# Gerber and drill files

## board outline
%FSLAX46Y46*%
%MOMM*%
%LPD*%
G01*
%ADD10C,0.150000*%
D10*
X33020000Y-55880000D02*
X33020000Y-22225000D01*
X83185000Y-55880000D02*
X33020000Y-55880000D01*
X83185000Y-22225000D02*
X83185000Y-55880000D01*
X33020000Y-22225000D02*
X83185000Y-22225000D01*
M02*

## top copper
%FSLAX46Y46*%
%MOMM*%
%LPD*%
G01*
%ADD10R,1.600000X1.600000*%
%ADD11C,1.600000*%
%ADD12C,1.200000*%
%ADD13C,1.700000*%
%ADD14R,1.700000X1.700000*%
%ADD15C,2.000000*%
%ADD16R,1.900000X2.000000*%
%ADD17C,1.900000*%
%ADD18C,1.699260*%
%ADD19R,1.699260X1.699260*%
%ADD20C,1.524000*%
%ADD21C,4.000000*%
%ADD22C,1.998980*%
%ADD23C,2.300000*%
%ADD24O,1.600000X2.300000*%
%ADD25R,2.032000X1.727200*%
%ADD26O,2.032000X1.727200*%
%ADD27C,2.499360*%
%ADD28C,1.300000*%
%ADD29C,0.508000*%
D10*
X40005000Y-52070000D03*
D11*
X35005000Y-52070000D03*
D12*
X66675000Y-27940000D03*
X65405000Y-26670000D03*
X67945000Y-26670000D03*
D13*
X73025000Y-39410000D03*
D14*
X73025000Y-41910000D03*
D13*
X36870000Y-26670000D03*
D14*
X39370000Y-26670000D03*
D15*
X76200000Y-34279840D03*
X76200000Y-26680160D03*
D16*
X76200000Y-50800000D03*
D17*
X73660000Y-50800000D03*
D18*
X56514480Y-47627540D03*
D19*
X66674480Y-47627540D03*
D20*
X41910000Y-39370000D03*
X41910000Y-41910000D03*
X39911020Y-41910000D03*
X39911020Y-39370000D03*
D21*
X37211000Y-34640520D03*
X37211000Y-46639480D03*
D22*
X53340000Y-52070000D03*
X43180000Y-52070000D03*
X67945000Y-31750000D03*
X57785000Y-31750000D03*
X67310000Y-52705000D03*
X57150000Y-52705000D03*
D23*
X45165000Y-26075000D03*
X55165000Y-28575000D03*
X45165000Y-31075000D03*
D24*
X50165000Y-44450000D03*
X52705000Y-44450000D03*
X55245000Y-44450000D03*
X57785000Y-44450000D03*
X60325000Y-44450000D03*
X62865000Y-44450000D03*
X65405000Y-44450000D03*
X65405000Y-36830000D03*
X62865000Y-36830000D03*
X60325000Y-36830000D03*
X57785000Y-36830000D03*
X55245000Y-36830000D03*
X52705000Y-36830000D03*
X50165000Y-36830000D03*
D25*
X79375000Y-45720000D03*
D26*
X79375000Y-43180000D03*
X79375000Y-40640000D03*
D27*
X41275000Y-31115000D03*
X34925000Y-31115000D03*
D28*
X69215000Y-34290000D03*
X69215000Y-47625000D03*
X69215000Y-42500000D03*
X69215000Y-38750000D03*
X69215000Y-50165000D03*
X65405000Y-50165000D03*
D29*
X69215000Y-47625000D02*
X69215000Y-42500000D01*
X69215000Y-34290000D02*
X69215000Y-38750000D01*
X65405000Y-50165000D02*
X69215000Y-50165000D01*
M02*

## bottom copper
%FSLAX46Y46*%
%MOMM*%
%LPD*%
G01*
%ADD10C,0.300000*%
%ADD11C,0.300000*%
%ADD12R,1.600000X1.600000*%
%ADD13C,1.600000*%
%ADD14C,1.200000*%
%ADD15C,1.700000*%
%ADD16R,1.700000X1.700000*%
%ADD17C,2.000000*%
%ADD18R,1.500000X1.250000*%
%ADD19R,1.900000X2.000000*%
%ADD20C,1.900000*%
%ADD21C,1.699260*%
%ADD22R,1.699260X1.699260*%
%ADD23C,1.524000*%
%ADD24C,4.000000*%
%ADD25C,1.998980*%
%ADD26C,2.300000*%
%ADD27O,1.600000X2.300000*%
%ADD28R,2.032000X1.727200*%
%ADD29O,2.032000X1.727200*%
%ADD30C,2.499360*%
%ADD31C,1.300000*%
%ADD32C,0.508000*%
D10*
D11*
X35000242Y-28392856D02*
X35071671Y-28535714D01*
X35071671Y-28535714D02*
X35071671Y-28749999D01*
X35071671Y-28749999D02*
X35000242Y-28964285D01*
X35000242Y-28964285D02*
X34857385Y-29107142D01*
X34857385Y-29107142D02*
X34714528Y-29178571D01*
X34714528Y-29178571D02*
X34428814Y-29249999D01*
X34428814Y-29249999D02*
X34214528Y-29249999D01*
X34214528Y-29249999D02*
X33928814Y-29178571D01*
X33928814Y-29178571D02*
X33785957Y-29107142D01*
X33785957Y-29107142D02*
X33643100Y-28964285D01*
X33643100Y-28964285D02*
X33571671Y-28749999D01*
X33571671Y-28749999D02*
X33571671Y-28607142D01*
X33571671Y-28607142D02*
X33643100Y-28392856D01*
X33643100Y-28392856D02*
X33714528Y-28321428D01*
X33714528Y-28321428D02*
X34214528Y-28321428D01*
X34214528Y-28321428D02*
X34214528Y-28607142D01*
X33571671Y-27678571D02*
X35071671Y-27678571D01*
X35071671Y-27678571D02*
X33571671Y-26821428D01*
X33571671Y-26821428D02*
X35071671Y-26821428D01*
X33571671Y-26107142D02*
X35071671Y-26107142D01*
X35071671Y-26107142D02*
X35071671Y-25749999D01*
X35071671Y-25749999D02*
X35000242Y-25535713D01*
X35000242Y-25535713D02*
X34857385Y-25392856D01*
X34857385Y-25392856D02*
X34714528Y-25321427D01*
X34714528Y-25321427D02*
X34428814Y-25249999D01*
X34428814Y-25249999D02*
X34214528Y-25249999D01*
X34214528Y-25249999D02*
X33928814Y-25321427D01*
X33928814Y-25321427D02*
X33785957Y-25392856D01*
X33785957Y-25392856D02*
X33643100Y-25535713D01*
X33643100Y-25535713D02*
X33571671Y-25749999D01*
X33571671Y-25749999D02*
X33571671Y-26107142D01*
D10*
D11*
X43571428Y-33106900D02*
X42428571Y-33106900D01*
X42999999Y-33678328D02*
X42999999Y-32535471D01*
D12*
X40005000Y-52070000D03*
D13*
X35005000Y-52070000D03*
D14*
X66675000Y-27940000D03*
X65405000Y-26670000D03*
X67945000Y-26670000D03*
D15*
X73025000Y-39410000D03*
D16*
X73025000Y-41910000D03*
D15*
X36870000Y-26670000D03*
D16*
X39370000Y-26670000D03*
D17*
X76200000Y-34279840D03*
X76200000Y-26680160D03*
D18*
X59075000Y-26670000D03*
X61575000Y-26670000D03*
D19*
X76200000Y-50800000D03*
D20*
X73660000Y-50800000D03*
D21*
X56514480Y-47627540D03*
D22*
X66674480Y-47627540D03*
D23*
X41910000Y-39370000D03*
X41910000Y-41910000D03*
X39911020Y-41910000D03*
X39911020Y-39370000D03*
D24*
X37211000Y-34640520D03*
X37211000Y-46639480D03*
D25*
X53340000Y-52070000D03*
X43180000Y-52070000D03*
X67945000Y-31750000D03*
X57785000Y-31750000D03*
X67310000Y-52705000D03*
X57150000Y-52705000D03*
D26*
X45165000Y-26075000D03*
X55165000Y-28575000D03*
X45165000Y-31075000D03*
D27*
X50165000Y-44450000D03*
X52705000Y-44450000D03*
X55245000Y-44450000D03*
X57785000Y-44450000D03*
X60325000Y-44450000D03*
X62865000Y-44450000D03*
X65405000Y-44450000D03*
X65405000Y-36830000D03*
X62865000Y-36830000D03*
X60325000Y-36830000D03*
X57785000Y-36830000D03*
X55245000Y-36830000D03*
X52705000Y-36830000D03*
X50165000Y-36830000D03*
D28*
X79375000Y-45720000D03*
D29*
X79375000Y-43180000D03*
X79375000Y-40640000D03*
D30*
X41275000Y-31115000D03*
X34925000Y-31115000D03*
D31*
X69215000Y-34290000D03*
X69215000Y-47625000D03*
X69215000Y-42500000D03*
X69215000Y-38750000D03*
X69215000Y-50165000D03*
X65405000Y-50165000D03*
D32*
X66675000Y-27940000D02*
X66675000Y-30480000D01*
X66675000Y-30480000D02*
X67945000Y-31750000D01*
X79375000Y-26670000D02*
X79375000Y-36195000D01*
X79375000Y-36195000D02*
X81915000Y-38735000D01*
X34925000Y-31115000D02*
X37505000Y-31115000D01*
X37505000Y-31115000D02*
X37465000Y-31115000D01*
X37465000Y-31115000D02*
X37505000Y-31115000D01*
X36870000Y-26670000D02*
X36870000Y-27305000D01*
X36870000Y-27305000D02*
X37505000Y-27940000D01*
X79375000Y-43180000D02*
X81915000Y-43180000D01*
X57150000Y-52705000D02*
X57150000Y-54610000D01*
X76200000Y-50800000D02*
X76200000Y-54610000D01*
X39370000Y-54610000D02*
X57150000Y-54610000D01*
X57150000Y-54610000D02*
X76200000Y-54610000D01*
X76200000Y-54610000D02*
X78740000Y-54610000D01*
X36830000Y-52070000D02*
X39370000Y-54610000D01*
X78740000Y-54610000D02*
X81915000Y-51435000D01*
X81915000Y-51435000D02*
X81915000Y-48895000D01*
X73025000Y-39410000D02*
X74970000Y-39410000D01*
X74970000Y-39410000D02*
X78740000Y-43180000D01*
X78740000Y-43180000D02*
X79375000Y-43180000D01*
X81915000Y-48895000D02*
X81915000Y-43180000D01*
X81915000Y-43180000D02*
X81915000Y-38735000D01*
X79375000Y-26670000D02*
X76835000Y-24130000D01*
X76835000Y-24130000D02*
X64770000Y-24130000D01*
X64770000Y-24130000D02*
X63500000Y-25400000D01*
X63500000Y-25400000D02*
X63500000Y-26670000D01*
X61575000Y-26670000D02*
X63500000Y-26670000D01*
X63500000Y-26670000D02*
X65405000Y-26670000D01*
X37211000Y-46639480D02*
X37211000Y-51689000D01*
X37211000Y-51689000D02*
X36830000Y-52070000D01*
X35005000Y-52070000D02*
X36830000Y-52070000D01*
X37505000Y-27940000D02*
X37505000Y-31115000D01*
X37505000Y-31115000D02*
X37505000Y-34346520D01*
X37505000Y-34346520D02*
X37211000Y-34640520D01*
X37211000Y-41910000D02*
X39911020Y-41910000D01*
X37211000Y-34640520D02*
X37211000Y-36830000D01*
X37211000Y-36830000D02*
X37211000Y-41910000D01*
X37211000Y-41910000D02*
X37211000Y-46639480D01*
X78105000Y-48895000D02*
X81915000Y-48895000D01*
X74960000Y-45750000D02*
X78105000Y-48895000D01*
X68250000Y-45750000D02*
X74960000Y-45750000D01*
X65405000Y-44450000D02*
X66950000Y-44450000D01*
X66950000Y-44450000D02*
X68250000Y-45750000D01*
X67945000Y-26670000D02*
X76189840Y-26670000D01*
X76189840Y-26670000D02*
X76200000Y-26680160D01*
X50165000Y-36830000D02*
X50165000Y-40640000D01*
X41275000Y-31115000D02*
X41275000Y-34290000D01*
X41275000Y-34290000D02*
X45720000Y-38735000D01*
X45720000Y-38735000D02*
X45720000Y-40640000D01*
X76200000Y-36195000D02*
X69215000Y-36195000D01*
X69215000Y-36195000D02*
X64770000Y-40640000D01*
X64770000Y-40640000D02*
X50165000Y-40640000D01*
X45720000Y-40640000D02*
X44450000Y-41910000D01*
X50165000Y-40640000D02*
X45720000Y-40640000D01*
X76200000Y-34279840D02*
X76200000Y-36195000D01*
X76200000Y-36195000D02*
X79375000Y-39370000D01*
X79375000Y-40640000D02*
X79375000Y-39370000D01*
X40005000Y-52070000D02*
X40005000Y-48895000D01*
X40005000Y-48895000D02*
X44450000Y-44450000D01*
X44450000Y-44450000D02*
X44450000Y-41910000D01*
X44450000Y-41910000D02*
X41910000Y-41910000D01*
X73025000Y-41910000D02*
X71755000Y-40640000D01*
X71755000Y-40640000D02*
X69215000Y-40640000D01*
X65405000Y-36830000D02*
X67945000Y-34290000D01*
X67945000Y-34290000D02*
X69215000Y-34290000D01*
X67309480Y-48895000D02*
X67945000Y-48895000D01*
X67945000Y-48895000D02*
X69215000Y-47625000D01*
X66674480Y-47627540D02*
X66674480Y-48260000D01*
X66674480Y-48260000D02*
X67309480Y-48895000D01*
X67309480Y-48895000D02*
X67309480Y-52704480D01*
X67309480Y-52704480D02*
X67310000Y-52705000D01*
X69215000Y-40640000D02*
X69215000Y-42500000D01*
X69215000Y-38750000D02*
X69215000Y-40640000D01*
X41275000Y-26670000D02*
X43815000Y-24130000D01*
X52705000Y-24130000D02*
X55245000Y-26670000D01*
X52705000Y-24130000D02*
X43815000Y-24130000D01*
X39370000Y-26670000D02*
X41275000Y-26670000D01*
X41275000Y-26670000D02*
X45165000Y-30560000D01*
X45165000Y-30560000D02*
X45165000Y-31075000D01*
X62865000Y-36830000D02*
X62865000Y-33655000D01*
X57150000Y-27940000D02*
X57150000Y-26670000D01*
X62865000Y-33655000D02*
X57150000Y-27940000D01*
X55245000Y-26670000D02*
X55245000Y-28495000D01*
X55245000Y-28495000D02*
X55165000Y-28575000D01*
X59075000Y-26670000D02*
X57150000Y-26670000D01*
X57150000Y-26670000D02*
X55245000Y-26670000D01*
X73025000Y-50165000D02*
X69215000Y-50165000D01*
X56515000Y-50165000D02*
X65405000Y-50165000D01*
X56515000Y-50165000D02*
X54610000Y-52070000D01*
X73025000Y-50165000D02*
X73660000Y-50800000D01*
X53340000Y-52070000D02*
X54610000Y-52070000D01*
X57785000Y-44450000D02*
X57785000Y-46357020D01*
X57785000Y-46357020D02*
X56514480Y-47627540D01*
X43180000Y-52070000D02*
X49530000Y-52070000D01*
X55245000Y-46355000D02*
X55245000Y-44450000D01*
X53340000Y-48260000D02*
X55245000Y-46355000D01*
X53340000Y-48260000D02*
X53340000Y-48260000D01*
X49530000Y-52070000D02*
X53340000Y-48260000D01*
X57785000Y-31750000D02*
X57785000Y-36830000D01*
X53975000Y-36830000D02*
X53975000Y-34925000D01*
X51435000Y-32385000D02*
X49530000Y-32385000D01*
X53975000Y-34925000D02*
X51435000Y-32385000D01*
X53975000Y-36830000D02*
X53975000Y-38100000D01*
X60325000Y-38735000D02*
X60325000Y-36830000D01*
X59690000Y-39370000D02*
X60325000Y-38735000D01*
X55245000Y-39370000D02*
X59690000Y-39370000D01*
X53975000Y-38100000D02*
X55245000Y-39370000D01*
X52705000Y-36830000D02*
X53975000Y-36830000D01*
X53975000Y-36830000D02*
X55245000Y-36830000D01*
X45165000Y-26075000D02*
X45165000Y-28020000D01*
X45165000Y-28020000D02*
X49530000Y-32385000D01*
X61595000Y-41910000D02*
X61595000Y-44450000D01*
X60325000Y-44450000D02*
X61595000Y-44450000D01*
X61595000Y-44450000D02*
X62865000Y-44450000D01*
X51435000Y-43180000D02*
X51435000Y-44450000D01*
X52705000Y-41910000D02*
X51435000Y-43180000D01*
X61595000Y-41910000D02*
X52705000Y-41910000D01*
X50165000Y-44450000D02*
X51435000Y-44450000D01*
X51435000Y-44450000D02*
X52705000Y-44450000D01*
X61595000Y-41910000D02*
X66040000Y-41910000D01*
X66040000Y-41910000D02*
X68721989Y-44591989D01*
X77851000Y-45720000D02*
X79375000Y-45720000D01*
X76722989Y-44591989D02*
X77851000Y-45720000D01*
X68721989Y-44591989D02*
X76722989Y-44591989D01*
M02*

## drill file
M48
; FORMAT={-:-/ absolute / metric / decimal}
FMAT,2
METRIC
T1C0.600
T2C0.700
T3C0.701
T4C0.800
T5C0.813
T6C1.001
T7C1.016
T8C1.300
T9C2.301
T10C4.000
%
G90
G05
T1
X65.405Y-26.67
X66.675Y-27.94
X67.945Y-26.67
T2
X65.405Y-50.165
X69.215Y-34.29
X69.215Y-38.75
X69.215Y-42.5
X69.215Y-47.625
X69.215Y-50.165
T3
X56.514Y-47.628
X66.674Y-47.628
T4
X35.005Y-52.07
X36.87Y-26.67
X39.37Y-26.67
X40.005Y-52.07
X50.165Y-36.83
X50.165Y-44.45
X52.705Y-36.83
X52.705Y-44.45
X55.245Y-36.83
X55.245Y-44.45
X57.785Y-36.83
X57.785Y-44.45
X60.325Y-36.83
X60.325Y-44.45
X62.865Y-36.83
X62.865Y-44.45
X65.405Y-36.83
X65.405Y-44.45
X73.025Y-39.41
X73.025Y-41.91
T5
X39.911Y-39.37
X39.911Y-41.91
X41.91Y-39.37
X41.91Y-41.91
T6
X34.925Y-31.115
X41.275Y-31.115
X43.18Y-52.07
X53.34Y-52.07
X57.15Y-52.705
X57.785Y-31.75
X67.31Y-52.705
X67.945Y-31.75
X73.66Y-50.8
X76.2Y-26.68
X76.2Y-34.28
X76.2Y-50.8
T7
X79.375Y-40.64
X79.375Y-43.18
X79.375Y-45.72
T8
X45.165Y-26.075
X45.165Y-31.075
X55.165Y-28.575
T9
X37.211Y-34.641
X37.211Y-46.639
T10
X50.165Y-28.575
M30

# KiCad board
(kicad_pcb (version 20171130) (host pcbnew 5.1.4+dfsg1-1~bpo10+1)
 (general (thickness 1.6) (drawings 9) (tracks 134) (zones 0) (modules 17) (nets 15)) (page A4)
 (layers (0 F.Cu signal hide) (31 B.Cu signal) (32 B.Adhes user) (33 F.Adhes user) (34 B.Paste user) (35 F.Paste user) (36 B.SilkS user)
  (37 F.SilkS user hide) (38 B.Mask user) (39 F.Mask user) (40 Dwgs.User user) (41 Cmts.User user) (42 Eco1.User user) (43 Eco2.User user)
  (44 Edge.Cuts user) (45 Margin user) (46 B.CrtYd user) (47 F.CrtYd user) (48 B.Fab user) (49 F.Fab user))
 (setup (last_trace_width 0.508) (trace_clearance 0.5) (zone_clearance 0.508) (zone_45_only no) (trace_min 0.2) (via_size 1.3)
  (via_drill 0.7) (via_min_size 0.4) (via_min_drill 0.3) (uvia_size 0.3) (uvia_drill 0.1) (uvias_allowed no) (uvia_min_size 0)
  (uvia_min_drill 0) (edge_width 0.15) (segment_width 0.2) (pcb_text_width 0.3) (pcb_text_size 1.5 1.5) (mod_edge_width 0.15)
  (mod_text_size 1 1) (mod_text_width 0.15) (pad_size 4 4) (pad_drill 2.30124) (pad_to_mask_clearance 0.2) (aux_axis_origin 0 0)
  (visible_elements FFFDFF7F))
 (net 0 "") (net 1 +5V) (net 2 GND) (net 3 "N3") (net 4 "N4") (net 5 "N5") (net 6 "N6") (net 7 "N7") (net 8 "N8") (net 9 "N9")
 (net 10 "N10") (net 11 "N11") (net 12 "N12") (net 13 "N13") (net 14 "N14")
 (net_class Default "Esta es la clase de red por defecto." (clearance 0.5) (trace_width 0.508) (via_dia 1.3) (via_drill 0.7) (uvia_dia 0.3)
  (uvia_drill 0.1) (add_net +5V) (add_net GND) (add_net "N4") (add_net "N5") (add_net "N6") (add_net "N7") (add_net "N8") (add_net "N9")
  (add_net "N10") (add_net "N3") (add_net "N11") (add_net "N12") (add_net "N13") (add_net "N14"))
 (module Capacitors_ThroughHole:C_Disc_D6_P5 (layer F.Cu) (at 40.005 52.07 180)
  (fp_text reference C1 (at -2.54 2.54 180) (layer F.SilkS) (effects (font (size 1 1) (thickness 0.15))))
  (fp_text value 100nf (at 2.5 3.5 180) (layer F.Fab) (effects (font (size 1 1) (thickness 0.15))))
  (pad 1 thru_hole rect (at 0 0 180) (size 1.6 1.6) (drill 0.8) (layers *.Cu *.Mask F.SilkS) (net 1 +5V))
  (pad 2 thru_hole circle (at 5 0 180) (size 1.6 1.6) (drill 0.8) (layers *.Cu *.Mask F.SilkS) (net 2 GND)))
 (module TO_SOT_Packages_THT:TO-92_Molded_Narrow (layer F.Cu) (at 67.945 26.67 180)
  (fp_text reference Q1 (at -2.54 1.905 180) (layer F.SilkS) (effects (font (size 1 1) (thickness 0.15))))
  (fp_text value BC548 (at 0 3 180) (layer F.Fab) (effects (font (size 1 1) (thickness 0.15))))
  (pad 2 thru_hole circle (at 1.27 -1.27 270) (size 1.2 1.2) (drill 0.6) (layers *.Cu *.Mask F.SilkS) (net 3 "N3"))
  (pad 3 thru_hole circle (at 2.54 0 270) (size 1.2 1.2) (drill 0.6) (layers *.Cu *.Mask F.SilkS) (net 2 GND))
  (pad 1 thru_hole circle (at 0 0 270) (size 1.2 1.2) (drill 0.6) (layers *.Cu *.Mask F.SilkS) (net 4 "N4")))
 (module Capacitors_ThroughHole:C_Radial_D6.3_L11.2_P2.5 (layer F.Cu) (at 73.025 41.91 90)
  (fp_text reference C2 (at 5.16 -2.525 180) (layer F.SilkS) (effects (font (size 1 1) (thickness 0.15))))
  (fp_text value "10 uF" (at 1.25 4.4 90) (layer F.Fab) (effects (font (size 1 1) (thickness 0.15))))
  (pad 2 thru_hole circle (at 2.5 0 90) (size 1.7 1.7) (drill 0.8) (layers *.Cu *.Mask F.SilkS) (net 2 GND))
  (pad 1 thru_hole rect (at 0 0 90) (size 1.7 1.7) (drill 0.8) (layers *.Cu *.Mask F.SilkS) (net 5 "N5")))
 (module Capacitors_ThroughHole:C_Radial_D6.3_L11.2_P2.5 (layer F.Cu) (at 39.37 26.67 180)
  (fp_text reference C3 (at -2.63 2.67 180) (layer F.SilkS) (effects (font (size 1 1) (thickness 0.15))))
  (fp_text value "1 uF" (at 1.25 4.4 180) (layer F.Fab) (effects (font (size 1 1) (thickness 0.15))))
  (pad 2 thru_hole circle (at 2.5 0 180) (size 1.7 1.7) (drill 0.8) (layers *.Cu *.Mask F.SilkS) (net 2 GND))
  (pad 1 thru_hole rect (at 0 0 180) (size 1.7 1.7) (drill 0.8) (layers *.Cu *.Mask F.SilkS) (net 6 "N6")))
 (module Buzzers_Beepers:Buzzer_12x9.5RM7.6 (layer F.Cu) (at 76.2 30.48 90)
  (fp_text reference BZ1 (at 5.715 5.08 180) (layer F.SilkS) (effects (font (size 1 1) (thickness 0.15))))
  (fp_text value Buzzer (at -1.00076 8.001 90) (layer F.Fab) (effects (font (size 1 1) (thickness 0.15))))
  (pad 1 thru_hole circle (at -3.79984 0 90) (size 2 2) (drill 1.00076) (layers *.Cu *.Mask F.SilkS) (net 1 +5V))
  (pad 2 thru_hole circle (at 3.79984 0 90) (size 2 2) (drill 1.00076) (layers *.Cu *.Mask F.SilkS) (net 4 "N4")))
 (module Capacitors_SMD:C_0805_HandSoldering (layer B.Cu) (at 60.325 26.67)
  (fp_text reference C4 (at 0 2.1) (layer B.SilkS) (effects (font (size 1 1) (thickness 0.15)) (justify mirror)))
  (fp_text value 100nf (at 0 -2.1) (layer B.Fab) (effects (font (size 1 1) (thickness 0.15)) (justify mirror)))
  (pad 1 smd rect (at -1.25 0) (size 1.5 1.25) (layers B.Cu B.Paste B.Mask) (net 6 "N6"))
  (pad 2 smd rect (at 1.25 0) (size 1.5 1.25) (layers B.Cu B.Paste B.Mask) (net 2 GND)))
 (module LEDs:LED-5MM (layer F.Cu) (at 76.2 50.8 180)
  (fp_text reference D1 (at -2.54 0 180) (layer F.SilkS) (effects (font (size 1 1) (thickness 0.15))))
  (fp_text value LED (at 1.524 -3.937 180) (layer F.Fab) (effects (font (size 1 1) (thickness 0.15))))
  (pad 1 thru_hole rect (at 0 0 270) (size 2 1.9) (drill 1.00076) (layers *.Cu *.Mask F.SilkS) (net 2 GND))
  (pad 2 thru_hole circle (at 2.54 0 180) (size 1.9 1.9) (drill 1.00076) (layers *.Cu *.Mask F.SilkS) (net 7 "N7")))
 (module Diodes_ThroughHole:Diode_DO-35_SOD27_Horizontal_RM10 (layer F.Cu) (at 66.675 47.625 180)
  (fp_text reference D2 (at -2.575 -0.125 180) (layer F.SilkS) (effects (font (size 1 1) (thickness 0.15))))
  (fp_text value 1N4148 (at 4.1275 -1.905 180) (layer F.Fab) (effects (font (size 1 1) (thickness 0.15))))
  (pad 2 thru_hole circle (at 10.16052 -0.00254) (size 1.69926 1.69926) (drill 0.70104) (layers *.Cu *.Mask F.SilkS) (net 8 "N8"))
  (pad 1 thru_hole rect (at 0.00052 -0.00254) (size 1.69926 1.69926) (drill 0.70104) (layers *.Cu *.Mask F.SilkS) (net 5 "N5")))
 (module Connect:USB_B (layer F.Cu) (at 41.91 41.91 180) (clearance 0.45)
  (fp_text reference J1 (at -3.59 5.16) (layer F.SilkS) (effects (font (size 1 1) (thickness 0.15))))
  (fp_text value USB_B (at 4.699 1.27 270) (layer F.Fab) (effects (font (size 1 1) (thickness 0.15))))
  (pad 2 thru_hole circle (at 0 2.54 90) (size 1.524 1.524) (drill 0.8128) (layers *.Cu *.Mask F.SilkS) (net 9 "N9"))
  (pad 1 thru_hole circle (at 0 0 90) (size 1.524 1.524) (drill 0.8128) (layers *.Cu *.Mask F.SilkS) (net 1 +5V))
  (pad 4 thru_hole circle (at 1.99898 0 90) (size 1.524 1.524) (drill 0.8128) (layers *.Cu *.Mask F.SilkS) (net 2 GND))
  (pad 3 thru_hole circle (at 1.99898 2.54 90) (size 1.524 1.524) (drill 0.8128) (layers *.Cu *.Mask F.SilkS) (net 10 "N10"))
  (pad 5 thru_hole circle (at 4.699 7.26948 90) (size 4 4) (drill 2.30124) (layers *.Cu *.Mask F.SilkS) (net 2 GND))
  (pad 5 thru_hole circle (at 4.699 -4.72948 90) (size 4 4) (drill 2.30124) (layers *.Cu *.Mask F.SilkS) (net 2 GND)))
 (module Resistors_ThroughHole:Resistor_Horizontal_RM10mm (layer F.Cu) (at 53.34 52.07 180)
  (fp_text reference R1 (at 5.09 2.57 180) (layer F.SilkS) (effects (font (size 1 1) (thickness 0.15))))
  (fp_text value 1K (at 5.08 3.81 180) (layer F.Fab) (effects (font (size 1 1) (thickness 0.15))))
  (pad 1 thru_hole circle (at 0 0 180) (size 1.99898 1.99898) (drill 1.00076) (layers *.Cu *.SilkS *.Mask) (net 7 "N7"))
  (pad 2 thru_hole circle (at 10.16 0 180) (size 1.99898 1.99898) (drill 1.00076) (layers *.Cu *.SilkS *.Mask) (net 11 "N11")))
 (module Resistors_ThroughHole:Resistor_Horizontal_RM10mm (layer F.Cu) (at 67.945 31.75 180)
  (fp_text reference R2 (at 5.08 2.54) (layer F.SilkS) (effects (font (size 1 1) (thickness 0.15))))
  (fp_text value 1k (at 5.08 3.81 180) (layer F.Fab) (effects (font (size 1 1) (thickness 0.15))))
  (pad 1 thru_hole circle (at 0 0 180) (size 1.99898 1.99898) (drill 1.00076) (layers *.Cu *.SilkS *.Mask) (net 3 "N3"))
  (pad 2 thru_hole circle (at 10.16 0 180) (size 1.99898 1.99898) (drill 1.00076) (layers *.Cu *.SilkS *.Mask) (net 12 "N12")))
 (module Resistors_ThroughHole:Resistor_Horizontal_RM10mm (layer F.Cu) (at 67.31 52.705 180)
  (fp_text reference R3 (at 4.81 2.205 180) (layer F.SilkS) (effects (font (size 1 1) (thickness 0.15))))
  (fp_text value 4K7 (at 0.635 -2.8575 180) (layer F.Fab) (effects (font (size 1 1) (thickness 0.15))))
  (pad 1 thru_hole circle (at 0 0 180) (size 1.99898 1.99898) (drill 1.00076) (layers *.Cu *.SilkS *.Mask) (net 5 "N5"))
  (pad 2 thru_hole circle (at 10.16 0 180) (size 1.99898 1.99898) (drill 1.00076) (layers *.Cu *.SilkS *.Mask) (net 2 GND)))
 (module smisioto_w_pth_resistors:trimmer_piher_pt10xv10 (layer F.Cu) (at 50.165 28.575 90)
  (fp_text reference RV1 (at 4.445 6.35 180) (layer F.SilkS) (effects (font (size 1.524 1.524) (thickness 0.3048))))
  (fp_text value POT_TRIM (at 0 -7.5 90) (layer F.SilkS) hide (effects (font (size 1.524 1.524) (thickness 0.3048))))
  (pad 1 thru_hole circle (at 2.5 -5 90) (size 2.3 2.3) (drill 1.3) (layers *.Cu *.Mask F.SilkS) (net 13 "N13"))
  (pad 2 thru_hole circle (at 0 5 90) (size 2.3 2.3) (drill 1.3) (layers *.Cu *.Mask F.SilkS) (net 6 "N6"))
  (pad 3 thru_hole circle (at -2.5 -5 90) (size 2.3 2.3) (drill 1.3) (layers *.Cu *.Mask F.SilkS) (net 6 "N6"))
  (pad "" np_thru_hole circle (at 0 0 90) (size 4 4) (drill 4) (layers *.Cu *.Mask F.SilkS)))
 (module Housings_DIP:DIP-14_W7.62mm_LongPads (layer F.Cu) (at 50.165 44.45 90)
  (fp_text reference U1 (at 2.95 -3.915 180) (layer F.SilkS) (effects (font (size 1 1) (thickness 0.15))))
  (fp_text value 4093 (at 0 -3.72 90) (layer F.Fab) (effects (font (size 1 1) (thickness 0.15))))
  (pad 1 thru_hole oval (at 0 0 90) (size 2.3 1.6) (drill 0.8) (layers *.Cu *.Mask F.SilkS) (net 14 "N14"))
  (pad 2 thru_hole oval (at 0 2.54 90) (size 2.3 1.6) (drill 0.8) (layers *.Cu *.Mask F.SilkS) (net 14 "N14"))
  (pad 3 thru_hole oval (at 0 5.08 90) (size 2.3 1.6) (drill 0.8) (layers *.Cu *.Mask F.SilkS) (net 11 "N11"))
  (pad 4 thru_hole oval (at 0 7.62 90) (size 2.3 1.6) (drill 0.8) (layers *.Cu *.Mask F.SilkS) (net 8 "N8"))
  (pad 5 thru_hole oval (at 0 10.16 90) (size 2.3 1.6) (drill 0.8) (layers *.Cu *.Mask F.SilkS) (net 14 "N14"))
  (pad 6 thru_hole oval (at 0 12.7 90) (size 2.3 1.6) (drill 0.8) (layers *.Cu *.Mask F.SilkS) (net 14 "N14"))
  (pad 7 thru_hole oval (at 0 15.24 90) (size 2.3 1.6) (drill 0.8) (layers *.Cu *.Mask F.SilkS) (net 2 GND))
  (pad 8 thru_hole oval (at 7.62 15.24 90) (size 2.3 1.6) (drill 0.8) (layers *.Cu *.Mask F.SilkS) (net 5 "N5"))
  (pad 9 thru_hole oval (at 7.62 12.7 90) (size 2.3 1.6) (drill 0.8) (layers *.Cu *.Mask F.SilkS) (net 6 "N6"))
  (pad 10 thru_hole oval (at 7.62 10.16 90) (size 2.3 1.6) (drill 0.8) (layers *.Cu *.Mask F.SilkS) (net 13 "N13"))
  (pad 11 thru_hole oval (at 7.62 7.62 90) (size 2.3 1.6) (drill 0.8) (layers *.Cu *.Mask F.SilkS) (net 12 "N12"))
  (pad 12 thru_hole oval (at 7.62 5.08 90) (size 2.3 1.6) (drill 0.8) (layers *.Cu *.Mask F.SilkS) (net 13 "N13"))
  (pad 13 thru_hole oval (at 7.62 2.54 90) (size 2.3 1.6) (drill 0.8) (layers *.Cu *.Mask F.SilkS) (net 13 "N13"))
  (pad 14 thru_hole oval (at 7.62 0 90) (size 2.3 1.6) (drill 0.8) (layers *.Cu *.Mask F.SilkS) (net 1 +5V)))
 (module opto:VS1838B (layer F.Cu) (at 79.375 45.72 180)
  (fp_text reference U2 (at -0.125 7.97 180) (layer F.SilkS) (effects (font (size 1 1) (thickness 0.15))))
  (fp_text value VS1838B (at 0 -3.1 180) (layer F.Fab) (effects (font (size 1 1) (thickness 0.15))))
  (pad 1 thru_hole rect (at 0 0 180) (size 2.032 1.7272) (drill 1.016) (layers *.Cu *.Mask F.SilkS) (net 14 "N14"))
  (pad 2 thru_hole oval (at 0 2.54 180) (size 2.032 1.7272) (drill 1.016) (layers *.Cu *.Mask F.SilkS) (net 2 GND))
  (pad 3 thru_hole oval (at 0 5.08 180) (size 2.032 1.7272) (drill 1.016) (layers *.Cu *.Mask F.SilkS) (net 1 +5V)))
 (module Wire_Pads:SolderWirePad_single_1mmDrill (layer F.Cu) (at 41.275 31.115)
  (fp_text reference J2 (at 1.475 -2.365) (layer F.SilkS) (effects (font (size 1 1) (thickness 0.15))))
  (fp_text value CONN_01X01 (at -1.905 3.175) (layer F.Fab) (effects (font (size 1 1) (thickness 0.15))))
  (pad 1 thru_hole circle (at 0 0) (size 2.49936 2.49936) (drill 1.00076) (layers *.Cu *.Mask F.SilkS) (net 1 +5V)))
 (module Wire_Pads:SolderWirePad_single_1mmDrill (layer F.Cu) (at 34.925 31.115)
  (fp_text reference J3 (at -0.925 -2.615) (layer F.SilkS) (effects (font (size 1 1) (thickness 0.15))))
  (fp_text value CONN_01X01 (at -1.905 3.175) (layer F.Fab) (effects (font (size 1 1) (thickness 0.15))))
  (pad 1 thru_hole circle (at 0 0) (size 2.49936 2.49936) (drill 1.00076) (layers *.Cu *.Mask F.SilkS) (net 2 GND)))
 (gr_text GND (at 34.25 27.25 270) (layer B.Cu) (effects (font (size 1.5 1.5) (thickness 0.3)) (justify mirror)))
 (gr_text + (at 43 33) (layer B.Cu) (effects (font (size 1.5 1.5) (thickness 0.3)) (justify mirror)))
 (gr_line (start 33.02 55.88) (end 33.02 22.225) (angle 90) (layer Edge.Cuts) (width 0.15))
 (gr_line (start 83.185 55.88) (end 33.02 55.88) (angle 90) (layer Edge.Cuts) (width 0.15))
 (gr_line (start 83.185 22.225) (end 83.185 55.88) (angle 90) (layer Edge.Cuts) (width 0.15))
 (gr_line (start 33.02 22.225) (end 83.185 22.225) (angle 90) (layer Edge.Cuts) (width 0.15))
 (segment (start 66.675 27.94) (end 66.675 30.48) (width 0.508) (layer B.Cu) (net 3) (status 10))
 (segment (start 66.675 30.48) (end 67.945 31.75) (width 0.508) (layer B.Cu) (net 3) (status 20))
 (segment (start 79.375 26.67) (end 79.375 36.195) (width 0.508) (layer B.Cu) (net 2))
 (segment (start 79.375 36.195) (end 81.915 38.735) (width 0.508) (layer B.Cu) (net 2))
 (segment (start 34.925 31.115) (end 37.505 31.115) (width 0.508) (layer B.Cu) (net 2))
 (segment (start 37.505 31.115) (end 37.465 31.115) (width 0.508) (layer B.Cu) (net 2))
 (segment (start 37.465 31.115) (end 37.505 31.115) (width 0.508) (layer B.Cu) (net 2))
 (segment (start 36.87 26.67) (end 36.87 27.305) (width 0.508) (layer B.Cu) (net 2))
 (segment (start 36.87 27.305) (end 37.505 27.94) (width 0.508) (layer B.Cu) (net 2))
 (segment (start 79.375 43.18) (end 81.915 43.18) (width 0.508) (layer B.Cu) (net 2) (status 10))
 (segment (start 57.15 52.705) (end 57.15 54.61) (width 0.508) (layer B.Cu) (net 2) (status 10))
 (segment (start 76.2 50.8) (end 76.2 54.61) (width 0.508) (layer B.Cu) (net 2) (status 10))
 (segment (start 39.37 54.61) (end 57.15 54.61) (width 0.508) (layer B.Cu) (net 2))
 (segment (start 57.15 54.61) (end 76.2 54.61) (width 0.508) (layer B.Cu) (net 2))
 (segment (start 76.2 54.61) (end 78.74 54.61) (width 0.508) (layer B.Cu) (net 2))
 (segment (start 36.83 52.07) (end 39.37 54.61) (width 0.508) (layer B.Cu) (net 2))
 (segment (start 78.74 54.61) (end 81.915 51.435) (width 0.508) (layer B.Cu) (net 2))
 (segment (start 81.915 51.435) (end 81.915 48.895) (width 0.508) (layer B.Cu) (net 2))
 (segment (start 73.025 39.41) (end 74.97 39.41) (width 0.508) (layer B.Cu) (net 2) (status 10))
 (segment (start 74.97 39.41) (end 78.74 43.18) (width 0.508) (layer B.Cu) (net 2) (status 20))
 (segment (start 78.74 43.18) (end 79.375 43.18) (width 0.508) (layer B.Cu) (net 2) (status 30))
 (segment (start 81.915 48.895) (end 81.915 43.18) (width 0.508) (layer B.Cu) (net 2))
 (segment (start 81.915 43.18) (end 81.915 38.735) (width 0.508) (layer B.Cu) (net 2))
 (segment (start 79.375 26.67) (end 76.835 24.13) (width 0.508) (layer B.Cu) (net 2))
 (segment (start 76.835 24.13) (end 64.77 24.13) (width 0.508) (layer B.Cu) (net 2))
 (segment (start 64.77 24.13) (end 63.5 25.4) (width 0.508) (layer B.Cu) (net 2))
 (segment (start 63.5 25.4) (end 63.5 26.67) (width 0.508) (layer B.Cu) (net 2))
 (segment (start 61.575 26.67) (end 63.5 26.67) (width 0.508) (layer B.Cu) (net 2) (status 10))
 (segment (start 63.5 26.67) (end 65.405 26.67) (width 0.508) (layer B.Cu) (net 2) (status 20))
 (segment (start 37.211 46.63948) (end 37.211 51.689) (width 0.508) (layer B.Cu) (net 2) (status 10))
 (segment (start 37.211 51.689) (end 36.83 52.07) (width 0.508) (layer B.Cu) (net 2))
 (segment (start 35.005 52.07) (end 36.83 52.07) (width 0.508) (layer B.Cu) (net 2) (status 10))
 (segment (start 37.505 27.94) (end 37.505 31.115) (width 0.508) (layer B.Cu) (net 2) (status 30))
 (segment (start 37.505 31.115) (end 37.505 34.34652) (width 0.508) (layer B.Cu) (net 2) (status 30))
 (segment (start 37.505 34.34652) (end 37.211 34.64052) (width 0.508) (layer B.Cu) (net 2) (status 30))
 (segment (start 37.211 41.91) (end 39.91102 41.91) (width 0.508) (layer B.Cu) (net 2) (status 20))
 (segment (start 37.211 34.64052) (end 37.211 36.83) (width 0.508) (layer B.Cu) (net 2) (status 10))
 (segment (start 37.211 36.83) (end 37.211 41.91) (width 0.508) (layer B.Cu) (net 2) (status 10))
 (segment (start 37.211 41.91) (end 37.211 46.63948) (width 0.508) (layer B.Cu) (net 2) (status 20))
 (segment (start 78.105 48.895) (end 81.915 48.895) (width 0.508) (layer B.Cu) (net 2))
 (segment (start 74.96 45.75) (end 78.105 48.895) (width 0.508) (layer B.Cu) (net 2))
 (segment (start 68.25 45.75) (end 74.96 45.75) (width 0.508) (layer B.Cu) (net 2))
 (segment (start 65.405 44.45) (end 66.95 44.45) (width 0.508) (layer B.Cu) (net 2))
 (segment (start 66.95 44.45) (end 68.25 45.75) (width 0.508) (layer B.Cu) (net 2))
 (segment (start 67.945 26.67) (end 76.18984 26.67) (width 0.508) (layer B.Cu) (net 4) (status 30))
 (segment (start 76.18984 26.67) (end 76.2 26.68016) (width 0.508) (layer B.Cu) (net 4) (status 30))
 (segment (start 50.165 36.83) (end 50.165 40.64) (width 0.508) (layer B.Cu) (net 1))
 (segment (start 41.275 31.115) (end 41.275 34.29) (width 0.508) (layer B.Cu) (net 1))
 (segment (start 41.275 34.29) (end 45.72 38.735) (width 0.508) (layer B.Cu) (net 1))
 (segment (start 45.72 38.735) (end 45.72 40.64) (width 0.508) (layer B.Cu) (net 1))
 (segment (start 76.2 36.195) (end 69.215 36.195) (width 0.508) (layer B.Cu) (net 1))
 (segment (start 69.215 36.195) (end 64.77 40.64) (width 0.508) (layer B.Cu) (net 1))
 (segment (start 64.77 40.64) (end 50.165 40.64) (width 0.508) (layer B.Cu) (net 1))
 (segment (start 45.72 40.64) (end 44.45 41.91) (width 0.508) (layer B.Cu) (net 1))
 (segment (start 50.165 40.64) (end 45.72 40.64) (width 0.508) (layer B.Cu) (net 1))
 (segment (start 76.2 34.27984) (end 76.2 36.195) (width 0.508) (layer B.Cu) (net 1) (status 10))
 (segment (start 76.2 36.195) (end 79.375 39.37) (width 0.508) (layer B.Cu) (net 1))
 (segment (start 79.375 40.64) (end 79.375 39.37) (width 0.508) (layer B.Cu) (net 1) (status 10))
 (segment (start 40.005 52.07) (end 40.005 48.895) (width 0.508) (layer B.Cu) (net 1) (status 10))
 (segment (start 40.005 48.895) (end 44.45 44.45) (width 0.508) (layer B.Cu) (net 1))
 (segment (start 44.45 44.45) (end 44.45 41.91) (width 0.508) (layer B.Cu) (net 1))
 (segment (start 44.45 41.91) (end 41.91 41.91) (width 0.508) (layer B.Cu) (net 1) (status 20))
 (segment (start 73.025 41.91) (end 71.755 40.64) (width 0.508) (layer B.Cu) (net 5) (status 10))
 (segment (start 71.755 40.64) (end 69.215 40.64) (width 0.508) (layer B.Cu) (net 5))
 (segment (start 65.405 36.83) (end 67.945 34.29) (width 0.508) (layer B.Cu) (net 5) (status 10))
 (via (at 69.215 34.29) (size 1.3) (drill 0.7) (layers F.Cu B.Cu) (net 5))
 (segment (start 67.945 34.29) (end 69.215 34.29) (width 0.508) (layer B.Cu) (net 5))
 (segment (start 67.30948 48.895) (end 67.945 48.895) (width 0.508) (layer B.Cu) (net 5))
 (via (at 69.215 47.625) (size 1.3) (drill 0.7) (layers F.Cu B.Cu) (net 5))
 (segment (start 67.945 48.895) (end 69.215 47.625) (width 0.508) (layer B.Cu) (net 5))
 (segment (start 66.67448 47.62754) (end 66.67448 48.26) (width 0.508) (layer B.Cu) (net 5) (status 30))
 (segment (start 66.67448 48.26) (end 67.30948 48.895) (width 0.508) (layer B.Cu) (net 5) (status 10))
 (segment (start 67.30948 48.895) (end 67.30948 52.70448) (width 0.508) (layer B.Cu) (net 5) (status 20))
 (segment (start 67.30948 52.70448) (end 67.31 52.705) (width 0.508) (layer B.Cu) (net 5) (status 30))
 (segment (start 69.215 47.625) (end 69.215 42.5) (width 0.508) (layer F.Cu) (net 5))
 (via (at 69.215 42.5) (size 1.3) (drill 0.7) (layers F.Cu B.Cu) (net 5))
 (segment (start 69.215 40.64) (end 69.215 42.5) (width 0.508) (layer B.Cu) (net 5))
 (segment (start 69.215 34.29) (end 69.215 38.75) (width 0.508) (layer F.Cu) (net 5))
 (via (at 69.215 38.75) (size 1.3) (drill 0.7) (layers F.Cu B.Cu) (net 5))
 (segment (start 69.215 38.75) (end 69.215 40.64) (width 0.508) (layer B.Cu) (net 5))
 (segment (start 41.275 26.67) (end 43.815 24.13) (width 0.508) (layer B.Cu) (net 6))
 (segment (start 52.705 24.13) (end 55.245 26.67) (width 0.508) (layer B.Cu) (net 6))
 (segment (start 52.705 24.13) (end 43.815 24.13) (width 0.508) (layer B.Cu) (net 6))
 (segment (start 39.37 26.67) (end 41.275 26.67) (width 0.508) (layer B.Cu) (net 6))
 (segment (start 41.275 26.67) (end 45.165 30.56) (width 0.508) (layer B.Cu) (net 6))
 (segment (start 45.165 30.56) (end 45.165 31.075) (width 0.508) (layer B.Cu) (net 6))
 (segment (start 62.865 36.83) (end 62.865 33.655) (width 0.508) (layer B.Cu) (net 6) (status 10))
 (segment (start 57.15 27.94) (end 57.15 26.67) (width 0.508) (layer B.Cu) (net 6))
 (segment (start 62.865 33.655) (end 57.15 27.94) (width 0.508) (layer B.Cu) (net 6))
 (segment (start 55.245 26.67) (end 55.245 28.495) (width 0.508) (layer B.Cu) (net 6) (status 20))
 (segment (start 55.245 28.495) (end 55.165 28.575) (width 0.508) (layer B.Cu) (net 6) (status 30))
 (segment (start 59.075 26.67) (end 57.15 26.67) (width 0.508) (layer B.Cu) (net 6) (status 10))
 (segment (start 57.15 26.67) (end 55.245 26.67) (width 0.508) (layer B.Cu) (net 6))
 (segment (start 73.025 50.165) (end 69.215 50.165) (width 0.508) (layer B.Cu) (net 7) (status 10))
 (via (at 69.215 50.165) (size 1.3) (drill 0.7) (layers F.Cu B.Cu) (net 7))
 (segment (start 65.405 50.165) (end 69.215 50.165) (width 0.508) (layer F.Cu) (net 7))
 (via (at 65.405 50.165) (size 1.3) (drill 0.7) (layers F.Cu B.Cu) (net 7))
 (segment (start 56.515 50.165) (end 65.405 50.165) (width 0.508) (layer B.Cu) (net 7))
 (segment (start 56.515 50.165) (end 54.61 52.07) (width 0.508) (layer B.Cu) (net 7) (status 20))
 (segment (start 73.025 50.165) (end 73.66 50.8) (width 0.508) (layer B.Cu) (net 7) (status 30))
 (segment (start 53.34 52.07) (end 54.61 52.07) (width 0.508) (layer B.Cu) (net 7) (status 400030))
 (segment (start 57.785 44.45) (end 57.785 46.35702) (width 0.508) (layer B.Cu) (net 8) (status 10))
 (segment (start 57.785 46.35702) (end 56.51448 47.62754) (width 0.508) (layer B.Cu) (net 8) (status 20))
 (segment (start 43.18 52.07) (end 49.53 52.07) (width 0.508) (layer B.Cu) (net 11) (status 400010))
 (segment (start 55.245 46.355) (end 55.245 44.45) (width 0.508) (layer B.Cu) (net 11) (status 20))
 (segment (start 53.34 48.26) (end 55.245 46.355) (width 0.508) (layer B.Cu) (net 11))
 (segment (start 53.34 48.26) (end 53.34 48.26) (width 0.508) (layer B.Cu) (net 11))
 (segment (start 49.53 52.07) (end 53.34 48.26) (width 0.508) (layer B.Cu) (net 11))
 (segment (start 57.785 31.75) (end 57.785 36.83) (width 0.508) (layer B.Cu) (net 12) (status 30))
 (segment (start 53.975 36.83) (end 53.975 34.925) (width 0.508) (layer B.Cu) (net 13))
 (segment (start 51.435 32.385) (end 49.53 32.385) (width 0.508) (layer B.Cu) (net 13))
 (segment (start 53.975 34.925) (end 51.435 32.385) (width 0.508) (layer B.Cu) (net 13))
 (segment (start 53.975 36.83) (end 53.975 38.1) (width 0.508) (layer B.Cu) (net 13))
 (segment (start 60.325 38.735) (end 60.325 36.83) (width 0.508) (layer B.Cu) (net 13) (status 20))
 (segment (start 59.69 39.37) (end 60.325 38.735) (width 0.508) (layer B.Cu) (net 13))
 (segment (start 55.245 39.37) (end 59.69 39.37) (width 0.508) (layer B.Cu) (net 13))
 (segment (start 53.975 38.1) (end 55.245 39.37) (width 0.508) (layer B.Cu) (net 13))
 (segment (start 52.705 36.83) (end 53.975 36.83) (width 0.508) (layer B.Cu) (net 13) (status 10))
 (segment (start 53.975 36.83) (end 55.245 36.83) (width 0.508) (layer B.Cu) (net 13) (status 20))
 (segment (start 45.165 26.075) (end 45.165 28.02) (width 0.508) (layer B.Cu) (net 13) (status 10))
 (segment (start 45.165 28.02) (end 49.53 32.385) (width 0.508) (layer B.Cu) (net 13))
 (segment (start 61.595 41.91) (end 61.595 44.45) (width 0.508) (layer B.Cu) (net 14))
 (segment (start 60.325 44.45) (end 61.595 44.45) (width 0.508) (layer B.Cu) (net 14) (status 10))
 (segment (start 61.595 44.45) (end 62.865 44.45) (width 0.508) (layer B.Cu) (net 14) (status 20))
 (segment (start 51.435 43.18) (end 51.435 44.45) (width 0.508) (layer B.Cu) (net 14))
 (segment (start 52.705 41.91) (end 51.435 43.18) (width 0.508) (layer B.Cu) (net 14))
 (segment (start 61.595 41.91) (end 52.705 41.91) (width 0.508) (layer B.Cu) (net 14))
 (segment (start 50.165 44.45) (end 51.435 44.45) (width 0.508) (layer B.Cu) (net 14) (status 10))
 (segment (start 51.435 44.45) (end 52.705 44.45) (width 0.508) (layer B.Cu) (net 14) (status 20))
 (segment (start 61.595 41.91) (end 66.04 41.91) (width 0.508) (layer B.Cu) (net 14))
 (segment (start 66.04 41.91) (end 68.721989 44.591989) (width 0.508) (layer B.Cu) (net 14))
 (segment (start 77.851 45.72) (end 79.375 45.72) (width 0.508) (layer B.Cu) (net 14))
 (segment (start 76.722989 44.591989) (end 77.851 45.72) (width 0.508) (layer B.Cu) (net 14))
 (segment (start 68.721989 44.591989) (end 76.722989 44.591989) (width 0.508) (layer B.Cu) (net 14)))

